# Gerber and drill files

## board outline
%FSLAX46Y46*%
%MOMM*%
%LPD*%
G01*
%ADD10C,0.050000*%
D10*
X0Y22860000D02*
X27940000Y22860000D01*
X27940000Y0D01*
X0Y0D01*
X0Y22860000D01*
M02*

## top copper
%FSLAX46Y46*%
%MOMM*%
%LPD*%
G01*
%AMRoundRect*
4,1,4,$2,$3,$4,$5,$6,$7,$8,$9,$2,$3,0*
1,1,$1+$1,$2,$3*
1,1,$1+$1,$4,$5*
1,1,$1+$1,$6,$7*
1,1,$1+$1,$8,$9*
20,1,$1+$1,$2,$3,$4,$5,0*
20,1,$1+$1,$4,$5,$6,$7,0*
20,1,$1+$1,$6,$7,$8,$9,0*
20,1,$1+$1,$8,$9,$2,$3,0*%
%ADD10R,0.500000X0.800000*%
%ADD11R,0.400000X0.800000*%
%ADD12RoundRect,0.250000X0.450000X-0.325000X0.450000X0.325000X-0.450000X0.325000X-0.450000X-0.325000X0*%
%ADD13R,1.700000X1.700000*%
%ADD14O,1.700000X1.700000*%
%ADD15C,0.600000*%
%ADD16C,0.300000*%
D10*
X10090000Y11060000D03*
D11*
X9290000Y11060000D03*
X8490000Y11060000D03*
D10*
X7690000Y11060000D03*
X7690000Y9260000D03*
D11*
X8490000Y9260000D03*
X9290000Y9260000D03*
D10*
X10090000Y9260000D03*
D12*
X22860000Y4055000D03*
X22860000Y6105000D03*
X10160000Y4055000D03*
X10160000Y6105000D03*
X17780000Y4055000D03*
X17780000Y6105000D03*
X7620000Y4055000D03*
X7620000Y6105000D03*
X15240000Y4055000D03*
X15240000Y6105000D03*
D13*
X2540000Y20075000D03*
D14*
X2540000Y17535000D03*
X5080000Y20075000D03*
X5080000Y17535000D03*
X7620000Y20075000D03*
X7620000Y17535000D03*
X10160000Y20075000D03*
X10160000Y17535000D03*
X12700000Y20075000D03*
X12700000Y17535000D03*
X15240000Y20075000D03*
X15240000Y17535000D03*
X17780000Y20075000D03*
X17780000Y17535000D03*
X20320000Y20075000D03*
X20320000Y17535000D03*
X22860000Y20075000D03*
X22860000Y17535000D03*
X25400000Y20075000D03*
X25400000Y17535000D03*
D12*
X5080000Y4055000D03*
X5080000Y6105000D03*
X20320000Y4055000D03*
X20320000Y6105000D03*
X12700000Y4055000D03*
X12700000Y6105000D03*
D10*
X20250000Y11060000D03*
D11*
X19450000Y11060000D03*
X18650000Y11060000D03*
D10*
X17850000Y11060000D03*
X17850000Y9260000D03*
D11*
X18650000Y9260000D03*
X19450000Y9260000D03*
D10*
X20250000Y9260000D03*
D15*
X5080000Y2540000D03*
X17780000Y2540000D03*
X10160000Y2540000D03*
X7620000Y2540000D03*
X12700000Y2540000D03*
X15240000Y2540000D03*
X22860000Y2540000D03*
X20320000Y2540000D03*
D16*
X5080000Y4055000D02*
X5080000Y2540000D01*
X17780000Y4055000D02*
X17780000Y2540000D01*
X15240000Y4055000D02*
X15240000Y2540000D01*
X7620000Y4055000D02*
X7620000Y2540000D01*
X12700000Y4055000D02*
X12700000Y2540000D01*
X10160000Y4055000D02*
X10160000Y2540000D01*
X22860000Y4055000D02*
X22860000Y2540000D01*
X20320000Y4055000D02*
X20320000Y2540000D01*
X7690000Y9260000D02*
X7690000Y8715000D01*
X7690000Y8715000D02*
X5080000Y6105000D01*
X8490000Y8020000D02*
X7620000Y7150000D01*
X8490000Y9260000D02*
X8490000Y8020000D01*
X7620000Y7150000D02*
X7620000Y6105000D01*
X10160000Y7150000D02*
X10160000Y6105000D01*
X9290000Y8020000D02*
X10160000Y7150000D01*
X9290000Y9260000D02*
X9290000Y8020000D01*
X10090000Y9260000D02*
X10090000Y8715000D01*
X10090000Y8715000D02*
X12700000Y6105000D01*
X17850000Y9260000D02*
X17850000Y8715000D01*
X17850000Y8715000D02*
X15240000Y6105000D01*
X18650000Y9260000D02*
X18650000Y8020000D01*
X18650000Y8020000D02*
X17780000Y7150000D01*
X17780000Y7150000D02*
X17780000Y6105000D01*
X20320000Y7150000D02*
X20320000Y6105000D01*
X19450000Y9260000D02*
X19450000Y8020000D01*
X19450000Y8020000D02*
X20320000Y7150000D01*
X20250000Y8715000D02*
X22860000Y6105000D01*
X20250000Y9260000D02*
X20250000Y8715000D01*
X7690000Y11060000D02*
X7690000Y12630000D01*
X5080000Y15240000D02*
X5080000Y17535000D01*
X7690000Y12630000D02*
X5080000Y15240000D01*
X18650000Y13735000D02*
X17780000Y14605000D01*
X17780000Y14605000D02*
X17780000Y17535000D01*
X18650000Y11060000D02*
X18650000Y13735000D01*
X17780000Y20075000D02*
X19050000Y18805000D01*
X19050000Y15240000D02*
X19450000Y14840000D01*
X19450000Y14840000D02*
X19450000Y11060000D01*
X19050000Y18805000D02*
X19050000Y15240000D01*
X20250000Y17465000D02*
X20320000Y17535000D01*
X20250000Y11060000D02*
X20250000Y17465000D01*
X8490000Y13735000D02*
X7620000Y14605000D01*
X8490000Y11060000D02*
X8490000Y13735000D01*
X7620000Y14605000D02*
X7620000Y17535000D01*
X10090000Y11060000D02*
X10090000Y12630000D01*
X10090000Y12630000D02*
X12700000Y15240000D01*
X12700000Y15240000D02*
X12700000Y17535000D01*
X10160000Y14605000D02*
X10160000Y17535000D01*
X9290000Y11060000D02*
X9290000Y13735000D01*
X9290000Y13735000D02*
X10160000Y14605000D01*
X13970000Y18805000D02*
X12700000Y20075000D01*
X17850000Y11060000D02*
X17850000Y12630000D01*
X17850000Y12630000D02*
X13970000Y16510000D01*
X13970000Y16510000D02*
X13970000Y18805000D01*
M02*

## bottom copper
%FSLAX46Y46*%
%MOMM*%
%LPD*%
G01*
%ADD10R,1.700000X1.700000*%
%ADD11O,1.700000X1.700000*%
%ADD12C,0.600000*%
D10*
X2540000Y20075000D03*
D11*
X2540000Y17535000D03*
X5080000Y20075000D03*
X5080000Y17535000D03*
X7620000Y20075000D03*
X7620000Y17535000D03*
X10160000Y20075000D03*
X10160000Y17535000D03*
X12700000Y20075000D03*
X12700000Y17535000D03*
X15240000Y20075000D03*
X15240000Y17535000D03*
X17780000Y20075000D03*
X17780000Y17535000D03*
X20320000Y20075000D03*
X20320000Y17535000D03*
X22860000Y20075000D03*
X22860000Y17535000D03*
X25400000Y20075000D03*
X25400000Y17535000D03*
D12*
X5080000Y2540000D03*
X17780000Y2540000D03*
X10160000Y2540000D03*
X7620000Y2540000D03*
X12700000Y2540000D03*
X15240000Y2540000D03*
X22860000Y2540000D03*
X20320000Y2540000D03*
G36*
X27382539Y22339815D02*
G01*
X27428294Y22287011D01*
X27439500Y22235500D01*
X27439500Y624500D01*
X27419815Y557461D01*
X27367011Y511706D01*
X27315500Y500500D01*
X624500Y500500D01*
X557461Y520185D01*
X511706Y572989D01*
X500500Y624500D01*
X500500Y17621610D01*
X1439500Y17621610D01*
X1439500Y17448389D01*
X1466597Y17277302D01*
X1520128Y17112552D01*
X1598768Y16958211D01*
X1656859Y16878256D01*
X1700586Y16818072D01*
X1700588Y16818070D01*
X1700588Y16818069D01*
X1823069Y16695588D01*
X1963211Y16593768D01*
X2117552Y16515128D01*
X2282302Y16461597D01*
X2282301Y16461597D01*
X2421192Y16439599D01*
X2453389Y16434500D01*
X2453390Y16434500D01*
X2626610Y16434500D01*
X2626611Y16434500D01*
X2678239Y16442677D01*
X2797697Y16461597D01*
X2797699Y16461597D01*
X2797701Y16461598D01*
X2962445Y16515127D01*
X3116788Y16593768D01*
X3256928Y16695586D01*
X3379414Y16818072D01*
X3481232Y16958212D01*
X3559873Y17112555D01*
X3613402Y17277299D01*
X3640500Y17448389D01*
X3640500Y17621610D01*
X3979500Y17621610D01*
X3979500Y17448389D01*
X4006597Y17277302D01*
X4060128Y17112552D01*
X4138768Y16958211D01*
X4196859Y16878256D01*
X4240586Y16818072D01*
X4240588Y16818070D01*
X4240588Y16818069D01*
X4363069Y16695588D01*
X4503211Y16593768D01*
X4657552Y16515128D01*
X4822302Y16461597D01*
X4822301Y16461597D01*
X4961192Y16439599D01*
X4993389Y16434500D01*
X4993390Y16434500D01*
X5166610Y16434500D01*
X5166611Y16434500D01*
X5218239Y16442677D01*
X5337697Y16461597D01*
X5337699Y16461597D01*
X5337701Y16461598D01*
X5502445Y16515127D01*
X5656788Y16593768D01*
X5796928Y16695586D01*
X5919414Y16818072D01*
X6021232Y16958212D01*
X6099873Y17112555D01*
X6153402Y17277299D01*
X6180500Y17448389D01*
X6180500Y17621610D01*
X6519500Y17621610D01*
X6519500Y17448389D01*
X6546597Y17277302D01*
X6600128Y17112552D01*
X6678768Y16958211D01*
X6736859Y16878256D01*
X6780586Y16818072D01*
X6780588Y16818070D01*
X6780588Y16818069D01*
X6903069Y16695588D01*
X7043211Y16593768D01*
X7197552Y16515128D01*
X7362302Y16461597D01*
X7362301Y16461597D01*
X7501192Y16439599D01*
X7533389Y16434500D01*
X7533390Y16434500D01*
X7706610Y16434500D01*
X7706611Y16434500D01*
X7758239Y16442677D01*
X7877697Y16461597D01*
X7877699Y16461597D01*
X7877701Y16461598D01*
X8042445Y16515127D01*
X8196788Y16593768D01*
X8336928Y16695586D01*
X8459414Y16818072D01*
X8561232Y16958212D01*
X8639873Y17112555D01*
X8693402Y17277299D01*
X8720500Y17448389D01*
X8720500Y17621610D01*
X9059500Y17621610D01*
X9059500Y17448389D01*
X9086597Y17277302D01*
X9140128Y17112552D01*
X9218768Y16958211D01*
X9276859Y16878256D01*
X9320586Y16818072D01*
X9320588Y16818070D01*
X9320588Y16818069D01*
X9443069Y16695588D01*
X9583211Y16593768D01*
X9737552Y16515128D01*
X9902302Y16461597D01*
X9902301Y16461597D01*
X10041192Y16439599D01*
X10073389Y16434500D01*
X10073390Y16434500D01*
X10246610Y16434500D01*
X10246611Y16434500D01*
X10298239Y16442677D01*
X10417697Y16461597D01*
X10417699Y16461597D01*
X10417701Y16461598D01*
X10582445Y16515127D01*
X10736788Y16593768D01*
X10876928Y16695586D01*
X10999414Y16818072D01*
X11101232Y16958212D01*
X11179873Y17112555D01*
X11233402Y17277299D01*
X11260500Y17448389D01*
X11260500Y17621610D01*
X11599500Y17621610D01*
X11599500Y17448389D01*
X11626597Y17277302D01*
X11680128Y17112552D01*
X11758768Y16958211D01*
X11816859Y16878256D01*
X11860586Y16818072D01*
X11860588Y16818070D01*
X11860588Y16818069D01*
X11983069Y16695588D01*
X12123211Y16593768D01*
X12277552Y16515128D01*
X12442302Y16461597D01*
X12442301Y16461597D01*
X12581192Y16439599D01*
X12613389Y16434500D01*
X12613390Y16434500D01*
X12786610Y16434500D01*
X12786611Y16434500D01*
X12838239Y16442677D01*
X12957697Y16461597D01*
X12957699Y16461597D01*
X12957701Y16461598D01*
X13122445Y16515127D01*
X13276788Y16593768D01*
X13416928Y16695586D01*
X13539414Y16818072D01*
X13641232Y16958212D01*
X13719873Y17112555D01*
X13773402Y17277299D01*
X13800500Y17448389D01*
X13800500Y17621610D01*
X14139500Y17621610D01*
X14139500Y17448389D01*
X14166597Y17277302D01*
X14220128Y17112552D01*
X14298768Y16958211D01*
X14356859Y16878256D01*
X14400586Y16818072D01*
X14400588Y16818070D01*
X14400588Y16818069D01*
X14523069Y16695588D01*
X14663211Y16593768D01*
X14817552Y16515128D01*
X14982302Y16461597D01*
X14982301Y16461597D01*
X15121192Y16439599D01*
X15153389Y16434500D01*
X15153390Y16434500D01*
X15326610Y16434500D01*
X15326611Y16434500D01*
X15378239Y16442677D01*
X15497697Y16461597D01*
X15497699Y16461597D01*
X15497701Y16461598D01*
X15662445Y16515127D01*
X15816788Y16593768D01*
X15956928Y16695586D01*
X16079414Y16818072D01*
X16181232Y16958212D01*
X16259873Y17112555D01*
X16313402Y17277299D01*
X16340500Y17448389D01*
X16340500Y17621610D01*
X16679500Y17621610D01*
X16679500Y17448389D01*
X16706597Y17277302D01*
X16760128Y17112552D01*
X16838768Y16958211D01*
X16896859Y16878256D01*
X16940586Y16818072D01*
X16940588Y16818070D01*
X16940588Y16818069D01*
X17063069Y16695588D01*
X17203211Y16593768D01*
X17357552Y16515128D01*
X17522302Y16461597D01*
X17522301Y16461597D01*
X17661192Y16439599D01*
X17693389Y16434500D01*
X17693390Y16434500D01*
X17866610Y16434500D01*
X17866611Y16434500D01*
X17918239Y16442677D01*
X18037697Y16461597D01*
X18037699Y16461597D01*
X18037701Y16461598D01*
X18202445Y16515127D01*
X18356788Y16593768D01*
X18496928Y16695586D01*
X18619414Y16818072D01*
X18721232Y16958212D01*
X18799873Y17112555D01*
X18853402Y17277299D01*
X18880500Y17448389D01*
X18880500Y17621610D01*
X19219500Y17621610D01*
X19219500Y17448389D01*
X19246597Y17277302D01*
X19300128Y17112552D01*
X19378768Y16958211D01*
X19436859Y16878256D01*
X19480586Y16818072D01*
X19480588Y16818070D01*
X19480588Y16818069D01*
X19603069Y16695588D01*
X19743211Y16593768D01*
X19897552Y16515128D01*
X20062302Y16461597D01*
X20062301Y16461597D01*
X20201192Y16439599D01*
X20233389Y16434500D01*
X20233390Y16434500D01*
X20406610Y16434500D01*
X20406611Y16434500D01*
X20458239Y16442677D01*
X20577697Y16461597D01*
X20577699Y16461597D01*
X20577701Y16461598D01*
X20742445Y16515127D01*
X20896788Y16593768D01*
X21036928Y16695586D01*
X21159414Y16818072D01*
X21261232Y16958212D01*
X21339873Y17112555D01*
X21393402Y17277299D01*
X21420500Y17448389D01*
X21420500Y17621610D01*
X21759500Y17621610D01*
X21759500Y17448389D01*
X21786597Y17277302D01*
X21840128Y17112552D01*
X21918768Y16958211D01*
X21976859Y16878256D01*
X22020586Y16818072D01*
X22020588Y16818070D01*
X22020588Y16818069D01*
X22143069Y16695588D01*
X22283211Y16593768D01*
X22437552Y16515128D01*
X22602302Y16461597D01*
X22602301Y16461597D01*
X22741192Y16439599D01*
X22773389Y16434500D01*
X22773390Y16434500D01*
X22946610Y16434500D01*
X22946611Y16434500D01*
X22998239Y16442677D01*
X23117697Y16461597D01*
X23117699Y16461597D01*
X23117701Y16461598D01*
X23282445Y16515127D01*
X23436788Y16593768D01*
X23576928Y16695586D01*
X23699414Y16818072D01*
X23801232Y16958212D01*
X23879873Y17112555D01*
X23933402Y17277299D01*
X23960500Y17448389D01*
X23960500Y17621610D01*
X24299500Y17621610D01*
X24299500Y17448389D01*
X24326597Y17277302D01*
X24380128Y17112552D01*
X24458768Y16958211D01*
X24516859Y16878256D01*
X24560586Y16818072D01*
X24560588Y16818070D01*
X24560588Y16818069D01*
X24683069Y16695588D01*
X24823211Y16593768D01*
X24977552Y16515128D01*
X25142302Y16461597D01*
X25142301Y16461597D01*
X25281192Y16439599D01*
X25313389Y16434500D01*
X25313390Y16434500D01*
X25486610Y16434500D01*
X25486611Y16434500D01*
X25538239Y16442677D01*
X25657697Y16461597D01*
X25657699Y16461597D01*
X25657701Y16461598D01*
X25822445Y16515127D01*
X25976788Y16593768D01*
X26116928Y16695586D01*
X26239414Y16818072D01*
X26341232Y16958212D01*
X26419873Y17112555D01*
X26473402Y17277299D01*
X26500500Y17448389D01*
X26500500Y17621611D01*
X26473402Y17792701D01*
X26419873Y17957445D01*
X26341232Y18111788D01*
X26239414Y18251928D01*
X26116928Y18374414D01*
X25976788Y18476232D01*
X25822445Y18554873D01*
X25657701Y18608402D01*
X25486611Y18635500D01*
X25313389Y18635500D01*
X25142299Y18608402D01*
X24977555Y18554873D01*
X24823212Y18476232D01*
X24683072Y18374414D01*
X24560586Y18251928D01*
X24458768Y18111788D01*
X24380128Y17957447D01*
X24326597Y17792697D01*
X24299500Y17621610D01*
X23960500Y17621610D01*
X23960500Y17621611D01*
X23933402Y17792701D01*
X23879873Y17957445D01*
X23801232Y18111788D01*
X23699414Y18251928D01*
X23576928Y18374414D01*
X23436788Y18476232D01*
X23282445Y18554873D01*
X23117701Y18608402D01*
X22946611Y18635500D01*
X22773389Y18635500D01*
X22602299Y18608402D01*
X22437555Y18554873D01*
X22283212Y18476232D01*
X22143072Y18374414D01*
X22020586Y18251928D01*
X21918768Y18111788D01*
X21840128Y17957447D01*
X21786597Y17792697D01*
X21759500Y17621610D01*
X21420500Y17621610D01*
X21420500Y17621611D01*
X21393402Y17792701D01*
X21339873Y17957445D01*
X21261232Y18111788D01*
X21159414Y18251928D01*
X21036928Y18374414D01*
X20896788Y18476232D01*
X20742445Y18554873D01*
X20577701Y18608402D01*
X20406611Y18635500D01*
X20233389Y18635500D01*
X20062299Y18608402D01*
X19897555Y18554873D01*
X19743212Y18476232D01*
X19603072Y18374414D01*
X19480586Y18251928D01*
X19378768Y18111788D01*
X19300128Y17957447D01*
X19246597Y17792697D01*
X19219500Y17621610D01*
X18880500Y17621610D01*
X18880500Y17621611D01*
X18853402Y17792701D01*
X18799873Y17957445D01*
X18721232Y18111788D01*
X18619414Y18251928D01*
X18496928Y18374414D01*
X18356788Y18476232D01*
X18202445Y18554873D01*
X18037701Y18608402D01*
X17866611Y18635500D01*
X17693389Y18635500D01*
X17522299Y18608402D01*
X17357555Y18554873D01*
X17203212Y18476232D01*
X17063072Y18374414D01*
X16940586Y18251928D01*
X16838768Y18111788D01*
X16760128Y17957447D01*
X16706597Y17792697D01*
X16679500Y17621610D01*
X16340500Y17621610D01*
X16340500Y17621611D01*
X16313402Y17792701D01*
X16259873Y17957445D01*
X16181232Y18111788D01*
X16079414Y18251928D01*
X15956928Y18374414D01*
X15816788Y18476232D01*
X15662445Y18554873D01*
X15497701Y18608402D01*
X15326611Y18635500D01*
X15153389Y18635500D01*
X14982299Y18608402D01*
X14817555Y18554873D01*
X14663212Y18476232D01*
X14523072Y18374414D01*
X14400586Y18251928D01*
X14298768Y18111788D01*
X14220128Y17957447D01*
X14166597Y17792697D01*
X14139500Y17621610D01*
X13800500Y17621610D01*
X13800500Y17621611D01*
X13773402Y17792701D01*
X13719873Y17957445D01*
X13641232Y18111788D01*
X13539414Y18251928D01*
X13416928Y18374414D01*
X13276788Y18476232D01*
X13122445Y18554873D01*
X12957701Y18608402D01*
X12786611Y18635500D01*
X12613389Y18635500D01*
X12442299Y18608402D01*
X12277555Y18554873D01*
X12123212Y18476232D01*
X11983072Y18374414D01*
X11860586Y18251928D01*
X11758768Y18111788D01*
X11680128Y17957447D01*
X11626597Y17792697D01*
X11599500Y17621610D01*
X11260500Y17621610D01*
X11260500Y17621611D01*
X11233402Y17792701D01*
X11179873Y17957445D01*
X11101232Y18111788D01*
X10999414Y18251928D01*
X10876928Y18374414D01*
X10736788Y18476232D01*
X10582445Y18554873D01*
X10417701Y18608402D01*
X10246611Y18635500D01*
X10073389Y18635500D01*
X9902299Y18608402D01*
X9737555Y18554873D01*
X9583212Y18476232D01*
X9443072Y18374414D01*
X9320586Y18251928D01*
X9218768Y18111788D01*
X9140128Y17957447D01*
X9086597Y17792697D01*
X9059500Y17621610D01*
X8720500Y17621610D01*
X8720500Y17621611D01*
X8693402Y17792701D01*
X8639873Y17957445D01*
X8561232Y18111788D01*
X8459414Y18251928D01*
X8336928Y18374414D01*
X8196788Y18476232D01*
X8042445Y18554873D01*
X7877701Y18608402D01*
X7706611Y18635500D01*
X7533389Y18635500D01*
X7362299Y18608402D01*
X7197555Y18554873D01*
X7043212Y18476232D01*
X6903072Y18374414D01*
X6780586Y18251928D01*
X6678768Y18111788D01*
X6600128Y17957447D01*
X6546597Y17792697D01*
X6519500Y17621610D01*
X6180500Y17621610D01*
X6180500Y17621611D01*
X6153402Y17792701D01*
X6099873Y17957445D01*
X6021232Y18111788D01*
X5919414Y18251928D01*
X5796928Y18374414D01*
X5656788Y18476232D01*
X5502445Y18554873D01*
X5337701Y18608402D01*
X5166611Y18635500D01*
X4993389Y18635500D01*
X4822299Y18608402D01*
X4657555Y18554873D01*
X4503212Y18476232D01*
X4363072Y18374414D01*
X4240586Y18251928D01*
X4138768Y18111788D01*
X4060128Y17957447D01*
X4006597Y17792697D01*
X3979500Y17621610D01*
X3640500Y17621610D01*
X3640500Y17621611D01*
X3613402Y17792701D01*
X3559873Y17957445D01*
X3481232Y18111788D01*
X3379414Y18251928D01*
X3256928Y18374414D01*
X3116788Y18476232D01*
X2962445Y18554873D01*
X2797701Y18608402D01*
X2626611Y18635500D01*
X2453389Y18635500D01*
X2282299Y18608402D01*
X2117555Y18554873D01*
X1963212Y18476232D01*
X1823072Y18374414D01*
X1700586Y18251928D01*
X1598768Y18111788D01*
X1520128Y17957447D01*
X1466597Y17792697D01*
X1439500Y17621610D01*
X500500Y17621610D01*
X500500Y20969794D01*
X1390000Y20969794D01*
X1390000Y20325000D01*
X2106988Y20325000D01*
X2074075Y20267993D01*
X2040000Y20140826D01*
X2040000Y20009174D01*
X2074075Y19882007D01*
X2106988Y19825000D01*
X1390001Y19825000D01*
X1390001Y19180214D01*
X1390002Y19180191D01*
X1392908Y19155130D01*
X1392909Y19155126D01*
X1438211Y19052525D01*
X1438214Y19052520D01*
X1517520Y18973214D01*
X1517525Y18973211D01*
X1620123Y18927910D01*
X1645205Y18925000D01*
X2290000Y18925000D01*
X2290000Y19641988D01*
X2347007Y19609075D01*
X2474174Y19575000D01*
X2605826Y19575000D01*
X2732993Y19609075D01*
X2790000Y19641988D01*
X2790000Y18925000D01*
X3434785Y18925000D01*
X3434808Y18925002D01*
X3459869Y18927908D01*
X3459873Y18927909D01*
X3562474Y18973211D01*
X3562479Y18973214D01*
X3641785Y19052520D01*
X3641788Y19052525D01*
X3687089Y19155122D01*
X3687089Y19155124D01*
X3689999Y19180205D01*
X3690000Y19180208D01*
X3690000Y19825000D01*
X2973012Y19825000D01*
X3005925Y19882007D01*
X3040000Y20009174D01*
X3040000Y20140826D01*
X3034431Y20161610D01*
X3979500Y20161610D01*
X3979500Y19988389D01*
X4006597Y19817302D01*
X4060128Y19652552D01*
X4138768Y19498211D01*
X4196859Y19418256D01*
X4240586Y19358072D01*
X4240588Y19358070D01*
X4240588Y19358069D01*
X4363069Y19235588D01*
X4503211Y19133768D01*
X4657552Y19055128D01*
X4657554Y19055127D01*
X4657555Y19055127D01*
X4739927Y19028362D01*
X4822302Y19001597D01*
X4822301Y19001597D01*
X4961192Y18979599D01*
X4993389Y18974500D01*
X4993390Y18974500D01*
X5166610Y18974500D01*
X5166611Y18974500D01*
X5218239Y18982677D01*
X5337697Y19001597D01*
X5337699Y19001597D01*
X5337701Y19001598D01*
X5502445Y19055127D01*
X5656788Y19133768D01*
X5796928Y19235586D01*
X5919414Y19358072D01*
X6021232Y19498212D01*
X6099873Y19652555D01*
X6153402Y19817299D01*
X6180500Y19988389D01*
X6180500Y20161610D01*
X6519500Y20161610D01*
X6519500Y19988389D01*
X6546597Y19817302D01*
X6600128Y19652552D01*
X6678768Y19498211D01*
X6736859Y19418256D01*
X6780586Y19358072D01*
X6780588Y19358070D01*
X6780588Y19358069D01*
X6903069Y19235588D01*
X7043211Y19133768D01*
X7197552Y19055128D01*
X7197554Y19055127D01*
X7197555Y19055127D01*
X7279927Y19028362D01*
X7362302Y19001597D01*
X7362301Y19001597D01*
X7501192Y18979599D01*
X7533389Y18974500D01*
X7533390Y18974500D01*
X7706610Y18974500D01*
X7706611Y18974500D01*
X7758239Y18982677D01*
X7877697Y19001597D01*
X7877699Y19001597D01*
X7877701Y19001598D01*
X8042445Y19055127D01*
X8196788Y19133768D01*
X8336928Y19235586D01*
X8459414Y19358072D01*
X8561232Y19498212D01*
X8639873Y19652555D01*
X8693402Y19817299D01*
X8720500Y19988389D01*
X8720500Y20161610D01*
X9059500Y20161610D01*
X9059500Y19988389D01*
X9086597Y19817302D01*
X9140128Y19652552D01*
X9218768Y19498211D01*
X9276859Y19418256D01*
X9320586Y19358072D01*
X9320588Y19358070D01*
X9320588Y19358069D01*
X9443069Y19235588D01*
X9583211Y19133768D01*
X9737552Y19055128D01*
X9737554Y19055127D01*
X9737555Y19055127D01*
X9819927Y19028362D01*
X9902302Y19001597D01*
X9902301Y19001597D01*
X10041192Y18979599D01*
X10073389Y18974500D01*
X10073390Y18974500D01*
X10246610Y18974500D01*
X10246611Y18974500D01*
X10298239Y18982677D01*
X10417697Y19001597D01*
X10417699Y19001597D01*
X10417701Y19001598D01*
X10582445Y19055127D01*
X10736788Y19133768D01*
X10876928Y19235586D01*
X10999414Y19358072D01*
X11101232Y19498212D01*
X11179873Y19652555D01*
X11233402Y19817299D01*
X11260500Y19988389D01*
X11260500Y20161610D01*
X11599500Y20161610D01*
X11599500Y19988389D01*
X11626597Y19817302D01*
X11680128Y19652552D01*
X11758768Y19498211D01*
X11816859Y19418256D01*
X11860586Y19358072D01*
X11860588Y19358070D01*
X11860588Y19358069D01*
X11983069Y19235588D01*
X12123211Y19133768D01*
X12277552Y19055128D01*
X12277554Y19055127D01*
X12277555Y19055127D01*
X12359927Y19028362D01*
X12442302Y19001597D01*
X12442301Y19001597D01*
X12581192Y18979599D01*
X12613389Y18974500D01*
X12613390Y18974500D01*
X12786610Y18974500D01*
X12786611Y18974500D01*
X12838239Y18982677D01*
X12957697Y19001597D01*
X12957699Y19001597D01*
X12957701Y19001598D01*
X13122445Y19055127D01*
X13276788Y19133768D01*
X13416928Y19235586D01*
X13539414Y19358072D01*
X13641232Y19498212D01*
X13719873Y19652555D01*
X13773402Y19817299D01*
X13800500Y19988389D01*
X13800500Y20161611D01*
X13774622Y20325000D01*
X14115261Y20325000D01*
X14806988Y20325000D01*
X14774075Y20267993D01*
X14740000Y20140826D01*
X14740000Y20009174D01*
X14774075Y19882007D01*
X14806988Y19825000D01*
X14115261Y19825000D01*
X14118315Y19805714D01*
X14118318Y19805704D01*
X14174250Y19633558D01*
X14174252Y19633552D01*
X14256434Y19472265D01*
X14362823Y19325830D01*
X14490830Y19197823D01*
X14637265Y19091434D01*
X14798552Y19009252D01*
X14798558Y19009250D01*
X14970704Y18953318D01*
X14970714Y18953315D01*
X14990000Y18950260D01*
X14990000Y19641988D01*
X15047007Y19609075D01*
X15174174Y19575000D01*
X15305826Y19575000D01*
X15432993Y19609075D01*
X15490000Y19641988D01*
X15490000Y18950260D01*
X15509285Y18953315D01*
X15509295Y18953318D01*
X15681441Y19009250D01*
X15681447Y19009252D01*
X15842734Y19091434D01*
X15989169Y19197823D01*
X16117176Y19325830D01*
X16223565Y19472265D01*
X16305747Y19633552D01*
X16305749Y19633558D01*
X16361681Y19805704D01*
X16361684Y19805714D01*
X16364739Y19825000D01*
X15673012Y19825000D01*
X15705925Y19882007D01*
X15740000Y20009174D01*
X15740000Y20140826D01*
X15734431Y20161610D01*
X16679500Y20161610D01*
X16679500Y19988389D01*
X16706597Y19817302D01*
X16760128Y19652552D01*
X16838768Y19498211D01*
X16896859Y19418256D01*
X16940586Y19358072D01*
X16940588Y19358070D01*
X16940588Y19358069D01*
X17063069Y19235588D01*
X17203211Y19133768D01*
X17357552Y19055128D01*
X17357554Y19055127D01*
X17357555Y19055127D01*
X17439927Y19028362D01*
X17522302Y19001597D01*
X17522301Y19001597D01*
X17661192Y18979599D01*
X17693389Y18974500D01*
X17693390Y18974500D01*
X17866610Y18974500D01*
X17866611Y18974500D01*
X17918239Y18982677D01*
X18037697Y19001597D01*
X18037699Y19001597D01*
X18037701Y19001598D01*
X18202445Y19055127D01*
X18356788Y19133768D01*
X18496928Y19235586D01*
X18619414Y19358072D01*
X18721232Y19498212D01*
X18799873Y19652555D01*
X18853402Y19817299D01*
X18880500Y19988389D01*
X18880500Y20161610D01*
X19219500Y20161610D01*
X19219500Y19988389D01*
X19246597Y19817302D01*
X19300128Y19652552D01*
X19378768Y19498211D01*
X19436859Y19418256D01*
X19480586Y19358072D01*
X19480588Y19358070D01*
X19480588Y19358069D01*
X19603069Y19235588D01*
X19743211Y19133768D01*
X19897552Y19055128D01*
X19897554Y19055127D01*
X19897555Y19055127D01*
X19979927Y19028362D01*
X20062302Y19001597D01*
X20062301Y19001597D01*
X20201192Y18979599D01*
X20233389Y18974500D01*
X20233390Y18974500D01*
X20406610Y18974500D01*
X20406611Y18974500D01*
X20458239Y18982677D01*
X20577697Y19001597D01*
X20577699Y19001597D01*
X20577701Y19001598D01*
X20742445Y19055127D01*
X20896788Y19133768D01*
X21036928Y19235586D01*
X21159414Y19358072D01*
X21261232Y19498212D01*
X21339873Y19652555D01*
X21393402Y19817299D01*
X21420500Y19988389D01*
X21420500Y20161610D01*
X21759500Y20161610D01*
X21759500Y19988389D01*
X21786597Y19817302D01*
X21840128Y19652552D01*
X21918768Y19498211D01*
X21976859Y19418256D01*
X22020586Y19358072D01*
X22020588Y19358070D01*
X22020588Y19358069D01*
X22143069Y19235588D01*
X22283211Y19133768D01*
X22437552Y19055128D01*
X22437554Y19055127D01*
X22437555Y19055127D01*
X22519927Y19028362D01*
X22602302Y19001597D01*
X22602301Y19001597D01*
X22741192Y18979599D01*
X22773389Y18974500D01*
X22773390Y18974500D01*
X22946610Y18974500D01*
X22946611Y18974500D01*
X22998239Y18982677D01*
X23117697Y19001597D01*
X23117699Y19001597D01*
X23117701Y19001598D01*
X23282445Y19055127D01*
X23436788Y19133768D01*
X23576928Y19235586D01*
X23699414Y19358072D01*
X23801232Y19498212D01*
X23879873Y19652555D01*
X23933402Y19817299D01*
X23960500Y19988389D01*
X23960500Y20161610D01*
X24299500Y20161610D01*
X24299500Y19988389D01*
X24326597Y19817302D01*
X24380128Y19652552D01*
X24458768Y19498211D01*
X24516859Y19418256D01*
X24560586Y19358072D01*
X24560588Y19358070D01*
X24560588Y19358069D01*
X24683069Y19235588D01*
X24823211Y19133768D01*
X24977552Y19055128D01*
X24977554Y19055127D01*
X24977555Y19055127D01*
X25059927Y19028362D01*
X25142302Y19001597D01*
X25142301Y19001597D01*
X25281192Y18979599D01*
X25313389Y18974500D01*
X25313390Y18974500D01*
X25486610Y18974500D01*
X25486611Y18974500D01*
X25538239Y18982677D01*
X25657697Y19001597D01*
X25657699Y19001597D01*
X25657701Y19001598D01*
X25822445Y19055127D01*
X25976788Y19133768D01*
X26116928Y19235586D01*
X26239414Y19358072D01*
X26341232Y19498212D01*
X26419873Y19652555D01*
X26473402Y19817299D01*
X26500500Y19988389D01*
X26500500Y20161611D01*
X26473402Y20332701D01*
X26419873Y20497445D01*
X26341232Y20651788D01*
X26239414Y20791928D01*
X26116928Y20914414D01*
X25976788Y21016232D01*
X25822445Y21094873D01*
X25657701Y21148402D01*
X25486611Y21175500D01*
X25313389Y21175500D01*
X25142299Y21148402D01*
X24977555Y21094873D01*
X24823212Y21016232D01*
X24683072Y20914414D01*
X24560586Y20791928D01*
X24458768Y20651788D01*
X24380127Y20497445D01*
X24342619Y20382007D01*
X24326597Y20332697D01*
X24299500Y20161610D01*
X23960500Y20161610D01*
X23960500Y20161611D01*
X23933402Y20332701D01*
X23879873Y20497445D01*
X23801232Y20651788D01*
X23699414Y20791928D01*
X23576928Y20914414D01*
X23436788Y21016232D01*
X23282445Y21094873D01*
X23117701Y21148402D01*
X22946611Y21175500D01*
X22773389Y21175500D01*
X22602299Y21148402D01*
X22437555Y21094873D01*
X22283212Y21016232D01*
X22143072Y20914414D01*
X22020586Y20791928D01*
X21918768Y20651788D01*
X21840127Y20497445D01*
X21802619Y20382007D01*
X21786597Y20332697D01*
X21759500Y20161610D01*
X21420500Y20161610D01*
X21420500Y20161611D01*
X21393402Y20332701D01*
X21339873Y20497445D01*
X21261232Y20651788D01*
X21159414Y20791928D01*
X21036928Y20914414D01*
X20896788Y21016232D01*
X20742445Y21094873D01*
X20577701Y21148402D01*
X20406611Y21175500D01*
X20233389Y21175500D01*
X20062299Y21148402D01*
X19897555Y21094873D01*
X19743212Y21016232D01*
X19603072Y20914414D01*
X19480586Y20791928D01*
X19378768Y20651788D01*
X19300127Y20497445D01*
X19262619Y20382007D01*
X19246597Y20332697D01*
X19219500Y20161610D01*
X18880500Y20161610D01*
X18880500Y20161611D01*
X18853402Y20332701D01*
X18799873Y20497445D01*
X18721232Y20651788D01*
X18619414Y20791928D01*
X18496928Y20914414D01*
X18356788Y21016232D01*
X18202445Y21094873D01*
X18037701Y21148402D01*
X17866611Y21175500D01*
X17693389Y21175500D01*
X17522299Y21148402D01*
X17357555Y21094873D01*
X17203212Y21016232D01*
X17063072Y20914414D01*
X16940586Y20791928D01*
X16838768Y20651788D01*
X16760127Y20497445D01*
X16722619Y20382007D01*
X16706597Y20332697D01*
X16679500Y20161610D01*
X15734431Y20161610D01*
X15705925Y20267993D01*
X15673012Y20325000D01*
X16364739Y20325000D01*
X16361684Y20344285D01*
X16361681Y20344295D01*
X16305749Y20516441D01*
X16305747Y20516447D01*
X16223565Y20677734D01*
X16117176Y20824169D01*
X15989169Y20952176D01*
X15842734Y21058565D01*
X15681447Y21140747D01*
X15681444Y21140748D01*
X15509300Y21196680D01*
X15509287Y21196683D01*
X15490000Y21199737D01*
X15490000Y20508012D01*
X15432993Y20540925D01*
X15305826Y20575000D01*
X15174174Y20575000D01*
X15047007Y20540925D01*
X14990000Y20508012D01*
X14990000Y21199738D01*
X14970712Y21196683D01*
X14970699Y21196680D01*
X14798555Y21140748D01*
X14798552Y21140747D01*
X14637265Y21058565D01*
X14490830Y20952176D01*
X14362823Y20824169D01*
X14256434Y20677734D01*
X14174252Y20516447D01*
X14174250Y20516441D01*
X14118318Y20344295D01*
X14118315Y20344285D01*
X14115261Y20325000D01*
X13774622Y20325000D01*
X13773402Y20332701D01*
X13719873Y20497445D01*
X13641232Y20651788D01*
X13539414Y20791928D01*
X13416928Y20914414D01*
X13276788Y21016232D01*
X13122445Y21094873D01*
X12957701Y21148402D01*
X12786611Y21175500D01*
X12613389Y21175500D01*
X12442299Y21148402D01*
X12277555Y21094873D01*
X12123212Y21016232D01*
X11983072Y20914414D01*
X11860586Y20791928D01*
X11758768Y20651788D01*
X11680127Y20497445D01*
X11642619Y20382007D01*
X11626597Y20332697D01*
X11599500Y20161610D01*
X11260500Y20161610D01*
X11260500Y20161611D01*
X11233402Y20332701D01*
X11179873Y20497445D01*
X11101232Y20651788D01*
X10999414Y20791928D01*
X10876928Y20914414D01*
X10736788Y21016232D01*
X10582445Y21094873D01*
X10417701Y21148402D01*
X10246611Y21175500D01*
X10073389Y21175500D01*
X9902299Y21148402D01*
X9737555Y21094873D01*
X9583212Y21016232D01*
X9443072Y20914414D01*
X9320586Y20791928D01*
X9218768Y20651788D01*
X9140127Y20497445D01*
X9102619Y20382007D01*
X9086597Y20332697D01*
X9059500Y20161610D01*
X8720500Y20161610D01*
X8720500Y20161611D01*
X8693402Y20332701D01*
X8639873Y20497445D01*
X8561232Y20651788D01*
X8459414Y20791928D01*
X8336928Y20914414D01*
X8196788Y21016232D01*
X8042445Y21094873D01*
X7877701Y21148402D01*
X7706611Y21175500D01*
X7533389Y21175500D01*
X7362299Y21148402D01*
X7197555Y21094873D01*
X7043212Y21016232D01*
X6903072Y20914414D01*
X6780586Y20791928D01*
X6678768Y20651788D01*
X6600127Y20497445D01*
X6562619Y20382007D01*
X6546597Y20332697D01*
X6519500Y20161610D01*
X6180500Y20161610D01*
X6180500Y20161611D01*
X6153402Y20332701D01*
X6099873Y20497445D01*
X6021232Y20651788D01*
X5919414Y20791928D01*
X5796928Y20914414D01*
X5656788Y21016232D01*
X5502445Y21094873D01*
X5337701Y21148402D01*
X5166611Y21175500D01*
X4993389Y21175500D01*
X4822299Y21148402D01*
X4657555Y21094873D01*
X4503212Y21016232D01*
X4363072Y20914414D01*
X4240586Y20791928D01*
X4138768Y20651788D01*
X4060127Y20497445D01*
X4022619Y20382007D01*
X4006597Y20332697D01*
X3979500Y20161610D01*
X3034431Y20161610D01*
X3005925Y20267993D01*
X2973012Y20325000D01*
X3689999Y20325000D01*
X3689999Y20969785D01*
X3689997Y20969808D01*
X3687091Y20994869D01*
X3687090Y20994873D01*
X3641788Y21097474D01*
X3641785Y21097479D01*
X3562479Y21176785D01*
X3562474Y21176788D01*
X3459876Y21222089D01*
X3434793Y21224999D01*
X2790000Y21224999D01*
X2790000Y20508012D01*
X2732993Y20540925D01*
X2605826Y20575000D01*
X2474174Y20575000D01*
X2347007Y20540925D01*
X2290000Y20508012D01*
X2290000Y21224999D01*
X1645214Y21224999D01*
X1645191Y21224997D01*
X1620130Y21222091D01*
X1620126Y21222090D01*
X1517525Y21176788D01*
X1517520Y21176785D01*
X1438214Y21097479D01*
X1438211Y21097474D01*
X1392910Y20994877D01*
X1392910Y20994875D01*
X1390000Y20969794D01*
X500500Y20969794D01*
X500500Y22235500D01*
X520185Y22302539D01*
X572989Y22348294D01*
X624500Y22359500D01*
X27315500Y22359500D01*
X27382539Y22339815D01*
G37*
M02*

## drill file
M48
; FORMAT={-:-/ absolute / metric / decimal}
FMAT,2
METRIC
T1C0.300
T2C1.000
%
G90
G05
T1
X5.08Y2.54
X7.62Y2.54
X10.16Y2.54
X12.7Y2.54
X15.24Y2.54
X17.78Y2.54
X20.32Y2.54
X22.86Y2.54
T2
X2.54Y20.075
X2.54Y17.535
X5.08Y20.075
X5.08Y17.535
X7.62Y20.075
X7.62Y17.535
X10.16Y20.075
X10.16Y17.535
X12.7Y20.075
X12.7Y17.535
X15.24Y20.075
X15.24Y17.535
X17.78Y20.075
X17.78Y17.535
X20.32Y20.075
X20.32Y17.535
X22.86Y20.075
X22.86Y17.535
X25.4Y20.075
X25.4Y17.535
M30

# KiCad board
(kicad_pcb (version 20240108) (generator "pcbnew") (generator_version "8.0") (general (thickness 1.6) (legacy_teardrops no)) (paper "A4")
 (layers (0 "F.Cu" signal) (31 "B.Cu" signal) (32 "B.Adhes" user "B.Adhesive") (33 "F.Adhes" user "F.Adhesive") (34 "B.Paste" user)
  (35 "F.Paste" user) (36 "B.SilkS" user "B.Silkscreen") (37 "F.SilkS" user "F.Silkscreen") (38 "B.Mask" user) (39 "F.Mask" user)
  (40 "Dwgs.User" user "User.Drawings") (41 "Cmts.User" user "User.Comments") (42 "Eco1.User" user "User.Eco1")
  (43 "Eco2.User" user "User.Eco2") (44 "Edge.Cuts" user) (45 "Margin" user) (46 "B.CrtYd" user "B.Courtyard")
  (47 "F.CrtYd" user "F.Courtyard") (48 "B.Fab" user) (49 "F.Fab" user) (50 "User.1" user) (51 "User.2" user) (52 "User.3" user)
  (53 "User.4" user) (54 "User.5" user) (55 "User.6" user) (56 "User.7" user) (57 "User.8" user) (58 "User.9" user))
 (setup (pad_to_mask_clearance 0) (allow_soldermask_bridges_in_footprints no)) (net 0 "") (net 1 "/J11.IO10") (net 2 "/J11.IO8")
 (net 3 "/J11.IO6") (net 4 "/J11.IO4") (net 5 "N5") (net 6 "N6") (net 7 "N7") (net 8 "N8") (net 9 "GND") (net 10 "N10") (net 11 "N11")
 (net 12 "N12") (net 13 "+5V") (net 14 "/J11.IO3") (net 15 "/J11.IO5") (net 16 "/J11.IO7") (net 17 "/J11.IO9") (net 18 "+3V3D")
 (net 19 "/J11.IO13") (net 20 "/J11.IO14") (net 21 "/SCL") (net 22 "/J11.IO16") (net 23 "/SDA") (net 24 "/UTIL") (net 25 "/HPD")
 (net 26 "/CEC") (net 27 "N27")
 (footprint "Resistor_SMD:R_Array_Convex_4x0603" (layer "F.Cu") (at 8.89 -10.16 -90)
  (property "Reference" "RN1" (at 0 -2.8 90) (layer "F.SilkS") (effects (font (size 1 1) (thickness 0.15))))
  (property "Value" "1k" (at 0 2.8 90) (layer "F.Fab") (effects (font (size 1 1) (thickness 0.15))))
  (pad "1" smd rect (at -0.9 -1.2 270) (size 0.8 0.5) (layers "F.Cu" "F.Paste" "F.Mask") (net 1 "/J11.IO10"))
  (pad "2" smd rect (at -0.9 -0.4 270) (size 0.8 0.4) (layers "F.Cu" "F.Paste" "F.Mask") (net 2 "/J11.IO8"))
  (pad "3" smd rect (at -0.9 0.4 270) (size 0.8 0.4) (layers "F.Cu" "F.Paste" "F.Mask") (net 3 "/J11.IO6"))
  (pad "4" smd rect (at -0.9 1.2 270) (size 0.8 0.5) (layers "F.Cu" "F.Paste" "F.Mask") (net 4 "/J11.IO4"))
  (pad "5" smd rect (at 0.9 1.2 270) (size 0.8 0.5) (layers "F.Cu" "F.Paste" "F.Mask") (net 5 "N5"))
  (pad "6" smd rect (at 0.9 0.4 270) (size 0.8 0.4) (layers "F.Cu" "F.Paste" "F.Mask") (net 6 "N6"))
  (pad "7" smd rect (at 0.9 -0.4 270) (size 0.8 0.4) (layers "F.Cu" "F.Paste" "F.Mask") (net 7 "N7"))
  (pad "8" smd rect (at 0.9 -1.2 270) (size 0.8 0.5) (layers "F.Cu" "F.Paste" "F.Mask") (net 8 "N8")))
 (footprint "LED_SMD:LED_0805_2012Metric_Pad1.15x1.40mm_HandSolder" (layer "F.Cu") (at 22.86 -5.08 90)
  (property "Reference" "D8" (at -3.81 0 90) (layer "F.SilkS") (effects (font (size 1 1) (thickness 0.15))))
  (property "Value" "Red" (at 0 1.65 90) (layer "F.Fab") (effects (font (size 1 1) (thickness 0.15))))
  (pad "1" smd roundrect (at -1.025 0 90) (size 1.15 1.4) (layers "F.Cu" "F.Paste" "F.Mask") (roundrect_rratio 0.217391) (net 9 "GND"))
  (pad "2" smd roundrect (at 1.025 0 90) (size 1.15 1.4) (layers "F.Cu" "F.Paste" "F.Mask") (roundrect_rratio 0.217391) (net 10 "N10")))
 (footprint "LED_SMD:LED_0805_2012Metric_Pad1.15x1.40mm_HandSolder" (layer "F.Cu") (at 10.16 -5.08 90)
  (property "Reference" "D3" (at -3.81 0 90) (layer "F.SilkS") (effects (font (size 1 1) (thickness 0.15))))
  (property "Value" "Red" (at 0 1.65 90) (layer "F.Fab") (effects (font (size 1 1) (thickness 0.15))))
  (pad "1" smd roundrect (at -1.025 0 90) (size 1.15 1.4) (layers "F.Cu" "F.Paste" "F.Mask") (roundrect_rratio 0.217391) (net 9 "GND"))
  (pad "2" smd roundrect (at 1.025 0 90) (size 1.15 1.4) (layers "F.Cu" "F.Paste" "F.Mask") (roundrect_rratio 0.217391) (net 7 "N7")))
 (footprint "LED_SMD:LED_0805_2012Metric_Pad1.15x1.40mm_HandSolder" (layer "F.Cu") (at 17.78 -5.08 90)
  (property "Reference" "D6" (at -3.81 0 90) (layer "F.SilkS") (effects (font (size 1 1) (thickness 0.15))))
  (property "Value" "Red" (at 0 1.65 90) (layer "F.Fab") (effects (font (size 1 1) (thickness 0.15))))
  (pad "1" smd roundrect (at -1.025 0 90) (size 1.15 1.4) (layers "F.Cu" "F.Paste" "F.Mask") (roundrect_rratio 0.217391) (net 9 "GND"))
  (pad "2" smd roundrect (at 1.025 0 90) (size 1.15 1.4) (layers "F.Cu" "F.Paste" "F.Mask") (roundrect_rratio 0.217391) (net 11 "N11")))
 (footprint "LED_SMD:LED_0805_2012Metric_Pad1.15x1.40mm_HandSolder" (layer "F.Cu") (at 7.62 -5.08 90)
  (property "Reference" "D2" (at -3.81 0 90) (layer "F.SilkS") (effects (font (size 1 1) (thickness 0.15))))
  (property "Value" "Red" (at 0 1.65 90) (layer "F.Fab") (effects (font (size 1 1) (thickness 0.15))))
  (pad "1" smd roundrect (at -1.025 0 90) (size 1.15 1.4) (layers "F.Cu" "F.Paste" "F.Mask") (roundrect_rratio 0.217391) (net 9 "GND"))
  (pad "2" smd roundrect (at 1.025 0 90) (size 1.15 1.4) (layers "F.Cu" "F.Paste" "F.Mask") (roundrect_rratio 0.217391) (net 6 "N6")))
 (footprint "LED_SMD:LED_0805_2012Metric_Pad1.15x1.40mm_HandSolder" (layer "F.Cu") (at 15.24 -5.08 90)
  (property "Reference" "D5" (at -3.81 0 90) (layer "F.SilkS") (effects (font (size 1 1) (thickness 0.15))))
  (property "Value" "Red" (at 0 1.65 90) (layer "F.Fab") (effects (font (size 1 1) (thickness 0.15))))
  (pad "1" smd roundrect (at -1.025 0 90) (size 1.15 1.4) (layers "F.Cu" "F.Paste" "F.Mask") (roundrect_rratio 0.217391) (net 9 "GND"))
  (pad "2" smd roundrect (at 1.025 0 90) (size 1.15 1.4) (layers "F.Cu" "F.Paste" "F.Mask") (roundrect_rratio 0.217391) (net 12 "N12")))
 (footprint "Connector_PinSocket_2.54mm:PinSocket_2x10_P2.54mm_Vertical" (layer "F.Cu") (at 2.54 -20.075 90)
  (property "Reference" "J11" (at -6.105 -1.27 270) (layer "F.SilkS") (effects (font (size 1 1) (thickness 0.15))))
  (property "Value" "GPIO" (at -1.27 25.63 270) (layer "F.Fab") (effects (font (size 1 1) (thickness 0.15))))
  (pad "1" thru_hole rect (at 0 0 90) (size 1.7 1.7) (drill 1) (layers "*.Cu" "*.Mask") (remove_unused_layers no) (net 9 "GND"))
  (pad "2" thru_hole oval (at -2.54 0 90) (size 1.7 1.7) (drill 1) (layers "*.Cu" "*.Mask") (remove_unused_layers no) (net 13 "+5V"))
  (pad "3" thru_hole oval (at 0 2.54 90) (size 1.7 1.7) (drill 1) (layers "*.Cu" "*.Mask") (remove_unused_layers no) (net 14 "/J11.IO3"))
  (pad "4" thru_hole oval (at -2.54 2.54 90) (size 1.7 1.7) (drill 1) (layers "*.Cu" "*.Mask") (remove_unused_layers no) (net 4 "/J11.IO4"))
  (pad "5" thru_hole oval (at 0 5.08 90) (size 1.7 1.7) (drill 1) (layers "*.Cu" "*.Mask") (remove_unused_layers no) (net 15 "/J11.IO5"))
  (pad "6" thru_hole oval (at -2.54 5.08 90) (size 1.7 1.7) (drill 1) (layers "*.Cu" "*.Mask") (remove_unused_layers no) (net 3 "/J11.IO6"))
  (pad "7" thru_hole oval (at 0 7.62 90) (size 1.7 1.7) (drill 1) (layers "*.Cu" "*.Mask") (remove_unused_layers no) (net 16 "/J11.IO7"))
  (pad "8" thru_hole oval (at -2.54 7.62 90) (size 1.7 1.7) (drill 1) (layers "*.Cu" "*.Mask") (remove_unused_layers no) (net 2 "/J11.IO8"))
  (pad "9" thru_hole oval (at 0 10.16 90) (size 1.7 1.7) (drill 1) (layers "*.Cu" "*.Mask") (remove_unused_layers no) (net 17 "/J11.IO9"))
  (pad "10" thru_hole oval (at -2.54 10.16 90) (size 1.7 1.7) (drill 1) (layers "*.Cu" "*.Mask") (remove_unused_layers no)
   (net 1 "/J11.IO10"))
  (pad "11" thru_hole oval (at 0 12.7 90) (size 1.7 1.7) (drill 1) (layers "*.Cu" "*.Mask") (remove_unused_layers no) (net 9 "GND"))
  (pad "12" thru_hole oval (at -2.54 12.7 90) (size 1.7 1.7) (drill 1) (layers "*.Cu" "*.Mask") (remove_unused_layers no) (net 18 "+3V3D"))
  (pad "13" thru_hole oval (at 0 15.24 90) (size 1.7 1.7) (drill 1) (layers "*.Cu" "*.Mask") (remove_unused_layers no) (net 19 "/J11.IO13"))
  (pad "14" thru_hole oval (at -2.54 15.24 90) (size 1.7 1.7) (drill 1) (layers "*.Cu" "*.Mask") (remove_unused_layers no)
   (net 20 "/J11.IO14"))
  (pad "15" thru_hole oval (at 0 17.78 90) (size 1.7 1.7) (drill 1) (layers "*.Cu" "*.Mask") (remove_unused_layers no) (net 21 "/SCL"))
  (pad "16" thru_hole oval (at -2.54 17.78 90) (size 1.7 1.7) (drill 1) (layers "*.Cu" "*.Mask") (remove_unused_layers no)
   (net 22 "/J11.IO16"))
  (pad "17" thru_hole oval (at 0 20.32 90) (size 1.7 1.7) (drill 1) (layers "*.Cu" "*.Mask") (remove_unused_layers no) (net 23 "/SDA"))
  (pad "18" thru_hole oval (at -2.54 20.32 90) (size 1.7 1.7) (drill 1) (layers "*.Cu" "*.Mask") (remove_unused_layers no) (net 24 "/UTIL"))
  (pad "19" thru_hole oval (at 0 22.86 90) (size 1.7 1.7) (drill 1) (layers "*.Cu" "*.Mask") (remove_unused_layers no) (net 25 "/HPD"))
  (pad "20" thru_hole oval (at -2.54 22.86 90) (size 1.7 1.7) (drill 1) (layers "*.Cu" "*.Mask") (remove_unused_layers no) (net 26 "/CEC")))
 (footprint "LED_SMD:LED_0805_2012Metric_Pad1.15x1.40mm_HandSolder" (layer "F.Cu") (at 5.08 -5.08 90)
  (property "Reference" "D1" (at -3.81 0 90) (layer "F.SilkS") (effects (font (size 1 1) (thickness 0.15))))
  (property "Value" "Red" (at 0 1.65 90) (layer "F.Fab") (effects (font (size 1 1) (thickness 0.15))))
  (pad "1" smd roundrect (at -1.025 0 90) (size 1.15 1.4) (layers "F.Cu" "F.Paste" "F.Mask") (roundrect_rratio 0.217391) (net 9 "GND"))
  (pad "2" smd roundrect (at 1.025 0 90) (size 1.15 1.4) (layers "F.Cu" "F.Paste" "F.Mask") (roundrect_rratio 0.217391) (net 5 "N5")))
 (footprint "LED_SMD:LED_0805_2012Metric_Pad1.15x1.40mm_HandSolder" (layer "F.Cu") (at 20.32 -5.08 90)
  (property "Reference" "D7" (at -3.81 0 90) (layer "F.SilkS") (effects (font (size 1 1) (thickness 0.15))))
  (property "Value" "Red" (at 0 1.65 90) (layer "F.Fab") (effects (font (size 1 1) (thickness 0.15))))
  (pad "1" smd roundrect (at -1.025 0 90) (size 1.15 1.4) (layers "F.Cu" "F.Paste" "F.Mask") (roundrect_rratio 0.217391) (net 9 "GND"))
  (pad "2" smd roundrect (at 1.025 0 90) (size 1.15 1.4) (layers "F.Cu" "F.Paste" "F.Mask") (roundrect_rratio 0.217391) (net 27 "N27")))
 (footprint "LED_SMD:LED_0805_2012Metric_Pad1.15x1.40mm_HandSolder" (layer "F.Cu") (at 12.7 -5.08 90)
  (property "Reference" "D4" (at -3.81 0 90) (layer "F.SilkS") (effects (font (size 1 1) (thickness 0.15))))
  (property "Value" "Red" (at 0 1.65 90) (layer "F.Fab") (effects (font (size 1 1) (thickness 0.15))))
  (pad "1" smd roundrect (at -1.025 0 90) (size 1.15 1.4) (layers "F.Cu" "F.Paste" "F.Mask") (roundrect_rratio 0.217391) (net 9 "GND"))
  (pad "2" smd roundrect (at 1.025 0 90) (size 1.15 1.4) (layers "F.Cu" "F.Paste" "F.Mask") (roundrect_rratio 0.217391) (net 8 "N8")))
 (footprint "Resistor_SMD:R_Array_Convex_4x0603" (layer "F.Cu") (at 19.05 -10.16 -90)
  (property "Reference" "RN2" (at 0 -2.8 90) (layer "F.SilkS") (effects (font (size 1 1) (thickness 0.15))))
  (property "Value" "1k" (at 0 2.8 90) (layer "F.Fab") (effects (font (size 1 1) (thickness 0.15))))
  (pad "1" smd rect (at -0.9 -1.2 270) (size 0.8 0.5) (layers "F.Cu" "F.Paste" "F.Mask") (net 22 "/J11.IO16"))
  (pad "2" smd rect (at -0.9 -0.4 270) (size 0.8 0.4) (layers "F.Cu" "F.Paste" "F.Mask") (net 19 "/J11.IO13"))
  (pad "3" smd rect (at -0.9 0.4 270) (size 0.8 0.4) (layers "F.Cu" "F.Paste" "F.Mask") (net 20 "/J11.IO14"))
  (pad "4" smd rect (at -0.9 1.2 270) (size 0.8 0.5) (layers "F.Cu" "F.Paste" "F.Mask") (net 17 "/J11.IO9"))
  (pad "5" smd rect (at 0.9 1.2 270) (size 0.8 0.5) (layers "F.Cu" "F.Paste" "F.Mask") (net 12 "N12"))
  (pad "6" smd rect (at 0.9 0.4 270) (size 0.8 0.4) (layers "F.Cu" "F.Paste" "F.Mask") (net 11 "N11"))
  (pad "7" smd rect (at 0.9 -0.4 270) (size 0.8 0.4) (layers "F.Cu" "F.Paste" "F.Mask") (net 27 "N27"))
  (pad "8" smd rect (at 0.9 -1.2 270) (size 0.8 0.5) (layers "F.Cu" "F.Paste" "F.Mask") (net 10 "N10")))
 (gr_rect (start 0 -22.86) (end 27.94 0) (stroke (width 0.05) (type default)) (fill none) (layer "Edge.Cuts"))
 (segment (start 5.08 -4.055) (end 5.08 -2.54) (width 0.3) (layer "F.Cu") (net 9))
 (segment (start 17.78 -4.055) (end 17.78 -2.54) (width 0.3) (layer "F.Cu") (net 9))
 (segment (start 15.24 -4.055) (end 15.24 -2.54) (width 0.3) (layer "F.Cu") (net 9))
 (segment (start 7.62 -4.055) (end 7.62 -2.54) (width 0.3) (layer "F.Cu") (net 9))
 (segment (start 12.7 -4.055) (end 12.7 -2.54) (width 0.3) (layer "F.Cu") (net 9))
 (segment (start 10.16 -4.055) (end 10.16 -2.54) (width 0.3) (layer "F.Cu") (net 9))
 (segment (start 22.86 -4.055) (end 22.86 -2.54) (width 0.3) (layer "F.Cu") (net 9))
 (segment (start 20.32 -4.055) (end 20.32 -2.54) (width 0.3) (layer "F.Cu") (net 9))
 (via (at 5.08 -2.54) (size 0.6) (drill 0.3) (layers "F.Cu" "B.Cu") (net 9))
 (via (at 17.78 -2.54) (size 0.6) (drill 0.3) (layers "F.Cu" "B.Cu") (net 9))
 (via (at 10.16 -2.54) (size 0.6) (drill 0.3) (layers "F.Cu" "B.Cu") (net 9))
 (via (at 7.62 -2.54) (size 0.6) (drill 0.3) (layers "F.Cu" "B.Cu") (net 9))
 (via (at 12.7 -2.54) (size 0.6) (drill 0.3) (layers "F.Cu" "B.Cu") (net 9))
 (via (at 15.24 -2.54) (size 0.6) (drill 0.3) (layers "F.Cu" "B.Cu") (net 9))
 (via (at 22.86 -2.54) (size 0.6) (drill 0.3) (layers "F.Cu" "B.Cu") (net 9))
 (via (at 20.32 -2.54) (size 0.6) (drill 0.3) (layers "F.Cu" "B.Cu") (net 9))
 (segment (start 7.69 -9.26) (end 7.69 -8.715) (width 0.3) (layer "F.Cu") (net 5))
 (segment (start 7.69 -8.715) (end 5.08 -6.105) (width 0.3) (layer "F.Cu") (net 5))
 (segment (start 8.49 -8.02) (end 7.62 -7.15) (width 0.3) (layer "F.Cu") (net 6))
 (segment (start 8.49 -9.26) (end 8.49 -8.02) (width 0.3) (layer "F.Cu") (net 6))
 (segment (start 7.62 -7.15) (end 7.62 -6.105) (width 0.3) (layer "F.Cu") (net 6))
 (segment (start 10.16 -7.15) (end 10.16 -6.105) (width 0.3) (layer "F.Cu") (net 7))
 (segment (start 9.29 -8.02) (end 10.16 -7.15) (width 0.3) (layer "F.Cu") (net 7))
 (segment (start 9.29 -9.26) (end 9.29 -8.02) (width 0.3) (layer "F.Cu") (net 7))
 (segment (start 10.09 -9.26) (end 10.09 -8.715) (width 0.3) (layer "F.Cu") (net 8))
 (segment (start 10.09 -8.715) (end 12.7 -6.105) (width 0.3) (layer "F.Cu") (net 8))
 (segment (start 17.85 -9.26) (end 17.85 -8.715) (width 0.3) (layer "F.Cu") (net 12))
 (segment (start 17.85 -8.715) (end 15.24 -6.105) (width 0.3) (layer "F.Cu") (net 12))
 (segment (start 18.65 -9.26) (end 18.65 -8.02) (width 0.3) (layer "F.Cu") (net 11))
 (segment (start 18.65 -8.02) (end 17.78 -7.15) (width 0.3) (layer "F.Cu") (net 11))
 (segment (start 17.78 -7.15) (end 17.78 -6.105) (width 0.3) (layer "F.Cu") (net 11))
 (segment (start 20.32 -7.15) (end 20.32 -6.105) (width 0.3) (layer "F.Cu") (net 27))
 (segment (start 19.45 -9.26) (end 19.45 -8.02) (width 0.3) (layer "F.Cu") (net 27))
 (segment (start 19.45 -8.02) (end 20.32 -7.15) (width 0.3) (layer "F.Cu") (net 27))
 (segment (start 20.25 -8.715) (end 22.86 -6.105) (width 0.3) (layer "F.Cu") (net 10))
 (segment (start 20.25 -9.26) (end 20.25 -8.715) (width 0.3) (layer "F.Cu") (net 10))
 (segment (start 7.69 -11.06) (end 7.69 -12.63) (width 0.3) (layer "F.Cu") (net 4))
 (segment (start 5.08 -15.24) (end 5.08 -17.535) (width 0.3) (layer "F.Cu") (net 4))
 (segment (start 7.69 -12.63) (end 5.08 -15.24) (width 0.3) (layer "F.Cu") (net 4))
 (segment (start 18.65 -13.735) (end 17.78 -14.605) (width 0.3) (layer "F.Cu") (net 20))
 (segment (start 17.78 -14.605) (end 17.78 -17.535) (width 0.3) (layer "F.Cu") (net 20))
 (segment (start 18.65 -11.06) (end 18.65 -13.735) (width 0.3) (layer "F.Cu") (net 20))
 (segment (start 17.78 -20.075) (end 19.05 -18.805) (width 0.3) (layer "F.Cu") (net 19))
 (segment (start 19.05 -15.24) (end 19.45 -14.84) (width 0.3) (layer "F.Cu") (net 19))
 (segment (start 19.45 -14.84) (end 19.45 -11.06) (width 0.3) (layer "F.Cu") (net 19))
 (segment (start 19.05 -18.805) (end 19.05 -15.24) (width 0.3) (layer "F.Cu") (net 19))
 (segment (start 20.25 -17.465) (end 20.32 -17.535) (width 0.3) (layer "F.Cu") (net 22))
 (segment (start 20.25 -11.06) (end 20.25 -17.465) (width 0.3) (layer "F.Cu") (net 22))
 (segment (start 8.49 -13.735) (end 7.62 -14.605) (width 0.3) (layer "F.Cu") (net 3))
 (segment (start 8.49 -11.06) (end 8.49 -13.735) (width 0.3) (layer "F.Cu") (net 3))
 (segment (start 7.62 -14.605) (end 7.62 -17.535) (width 0.3) (layer "F.Cu") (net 3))
 (segment (start 10.09 -11.06) (end 10.09 -12.63) (width 0.3) (layer "F.Cu") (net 1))
 (segment (start 10.09 -12.63) (end 12.7 -15.24) (width 0.3) (layer "F.Cu") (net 1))
 (segment (start 12.7 -15.24) (end 12.7 -17.535) (width 0.3) (layer "F.Cu") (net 1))
 (segment (start 10.16 -14.605) (end 10.16 -17.535) (width 0.3) (layer "F.Cu") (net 2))
 (segment (start 9.29 -11.06) (end 9.29 -13.735) (width 0.3) (layer "F.Cu") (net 2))
 (segment (start 9.29 -13.735) (end 10.16 -14.605) (width 0.3) (layer "F.Cu") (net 2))
 (segment (start 13.97 -18.805) (end 12.7 -20.075) (width 0.3) (layer "F.Cu") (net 17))
 (segment (start 17.85 -11.06) (end 17.85 -12.63) (width 0.3) (layer "F.Cu") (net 17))
 (segment (start 17.85 -12.63) (end 13.97 -16.51) (width 0.3) (layer "F.Cu") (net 17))
 (segment (start 13.97 -16.51) (end 13.97 -18.805) (width 0.3) (layer "F.Cu") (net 17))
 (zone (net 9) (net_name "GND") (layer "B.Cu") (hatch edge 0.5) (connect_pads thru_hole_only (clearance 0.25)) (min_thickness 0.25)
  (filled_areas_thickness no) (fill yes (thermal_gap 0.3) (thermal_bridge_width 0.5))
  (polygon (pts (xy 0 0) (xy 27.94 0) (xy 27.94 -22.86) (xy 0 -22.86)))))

